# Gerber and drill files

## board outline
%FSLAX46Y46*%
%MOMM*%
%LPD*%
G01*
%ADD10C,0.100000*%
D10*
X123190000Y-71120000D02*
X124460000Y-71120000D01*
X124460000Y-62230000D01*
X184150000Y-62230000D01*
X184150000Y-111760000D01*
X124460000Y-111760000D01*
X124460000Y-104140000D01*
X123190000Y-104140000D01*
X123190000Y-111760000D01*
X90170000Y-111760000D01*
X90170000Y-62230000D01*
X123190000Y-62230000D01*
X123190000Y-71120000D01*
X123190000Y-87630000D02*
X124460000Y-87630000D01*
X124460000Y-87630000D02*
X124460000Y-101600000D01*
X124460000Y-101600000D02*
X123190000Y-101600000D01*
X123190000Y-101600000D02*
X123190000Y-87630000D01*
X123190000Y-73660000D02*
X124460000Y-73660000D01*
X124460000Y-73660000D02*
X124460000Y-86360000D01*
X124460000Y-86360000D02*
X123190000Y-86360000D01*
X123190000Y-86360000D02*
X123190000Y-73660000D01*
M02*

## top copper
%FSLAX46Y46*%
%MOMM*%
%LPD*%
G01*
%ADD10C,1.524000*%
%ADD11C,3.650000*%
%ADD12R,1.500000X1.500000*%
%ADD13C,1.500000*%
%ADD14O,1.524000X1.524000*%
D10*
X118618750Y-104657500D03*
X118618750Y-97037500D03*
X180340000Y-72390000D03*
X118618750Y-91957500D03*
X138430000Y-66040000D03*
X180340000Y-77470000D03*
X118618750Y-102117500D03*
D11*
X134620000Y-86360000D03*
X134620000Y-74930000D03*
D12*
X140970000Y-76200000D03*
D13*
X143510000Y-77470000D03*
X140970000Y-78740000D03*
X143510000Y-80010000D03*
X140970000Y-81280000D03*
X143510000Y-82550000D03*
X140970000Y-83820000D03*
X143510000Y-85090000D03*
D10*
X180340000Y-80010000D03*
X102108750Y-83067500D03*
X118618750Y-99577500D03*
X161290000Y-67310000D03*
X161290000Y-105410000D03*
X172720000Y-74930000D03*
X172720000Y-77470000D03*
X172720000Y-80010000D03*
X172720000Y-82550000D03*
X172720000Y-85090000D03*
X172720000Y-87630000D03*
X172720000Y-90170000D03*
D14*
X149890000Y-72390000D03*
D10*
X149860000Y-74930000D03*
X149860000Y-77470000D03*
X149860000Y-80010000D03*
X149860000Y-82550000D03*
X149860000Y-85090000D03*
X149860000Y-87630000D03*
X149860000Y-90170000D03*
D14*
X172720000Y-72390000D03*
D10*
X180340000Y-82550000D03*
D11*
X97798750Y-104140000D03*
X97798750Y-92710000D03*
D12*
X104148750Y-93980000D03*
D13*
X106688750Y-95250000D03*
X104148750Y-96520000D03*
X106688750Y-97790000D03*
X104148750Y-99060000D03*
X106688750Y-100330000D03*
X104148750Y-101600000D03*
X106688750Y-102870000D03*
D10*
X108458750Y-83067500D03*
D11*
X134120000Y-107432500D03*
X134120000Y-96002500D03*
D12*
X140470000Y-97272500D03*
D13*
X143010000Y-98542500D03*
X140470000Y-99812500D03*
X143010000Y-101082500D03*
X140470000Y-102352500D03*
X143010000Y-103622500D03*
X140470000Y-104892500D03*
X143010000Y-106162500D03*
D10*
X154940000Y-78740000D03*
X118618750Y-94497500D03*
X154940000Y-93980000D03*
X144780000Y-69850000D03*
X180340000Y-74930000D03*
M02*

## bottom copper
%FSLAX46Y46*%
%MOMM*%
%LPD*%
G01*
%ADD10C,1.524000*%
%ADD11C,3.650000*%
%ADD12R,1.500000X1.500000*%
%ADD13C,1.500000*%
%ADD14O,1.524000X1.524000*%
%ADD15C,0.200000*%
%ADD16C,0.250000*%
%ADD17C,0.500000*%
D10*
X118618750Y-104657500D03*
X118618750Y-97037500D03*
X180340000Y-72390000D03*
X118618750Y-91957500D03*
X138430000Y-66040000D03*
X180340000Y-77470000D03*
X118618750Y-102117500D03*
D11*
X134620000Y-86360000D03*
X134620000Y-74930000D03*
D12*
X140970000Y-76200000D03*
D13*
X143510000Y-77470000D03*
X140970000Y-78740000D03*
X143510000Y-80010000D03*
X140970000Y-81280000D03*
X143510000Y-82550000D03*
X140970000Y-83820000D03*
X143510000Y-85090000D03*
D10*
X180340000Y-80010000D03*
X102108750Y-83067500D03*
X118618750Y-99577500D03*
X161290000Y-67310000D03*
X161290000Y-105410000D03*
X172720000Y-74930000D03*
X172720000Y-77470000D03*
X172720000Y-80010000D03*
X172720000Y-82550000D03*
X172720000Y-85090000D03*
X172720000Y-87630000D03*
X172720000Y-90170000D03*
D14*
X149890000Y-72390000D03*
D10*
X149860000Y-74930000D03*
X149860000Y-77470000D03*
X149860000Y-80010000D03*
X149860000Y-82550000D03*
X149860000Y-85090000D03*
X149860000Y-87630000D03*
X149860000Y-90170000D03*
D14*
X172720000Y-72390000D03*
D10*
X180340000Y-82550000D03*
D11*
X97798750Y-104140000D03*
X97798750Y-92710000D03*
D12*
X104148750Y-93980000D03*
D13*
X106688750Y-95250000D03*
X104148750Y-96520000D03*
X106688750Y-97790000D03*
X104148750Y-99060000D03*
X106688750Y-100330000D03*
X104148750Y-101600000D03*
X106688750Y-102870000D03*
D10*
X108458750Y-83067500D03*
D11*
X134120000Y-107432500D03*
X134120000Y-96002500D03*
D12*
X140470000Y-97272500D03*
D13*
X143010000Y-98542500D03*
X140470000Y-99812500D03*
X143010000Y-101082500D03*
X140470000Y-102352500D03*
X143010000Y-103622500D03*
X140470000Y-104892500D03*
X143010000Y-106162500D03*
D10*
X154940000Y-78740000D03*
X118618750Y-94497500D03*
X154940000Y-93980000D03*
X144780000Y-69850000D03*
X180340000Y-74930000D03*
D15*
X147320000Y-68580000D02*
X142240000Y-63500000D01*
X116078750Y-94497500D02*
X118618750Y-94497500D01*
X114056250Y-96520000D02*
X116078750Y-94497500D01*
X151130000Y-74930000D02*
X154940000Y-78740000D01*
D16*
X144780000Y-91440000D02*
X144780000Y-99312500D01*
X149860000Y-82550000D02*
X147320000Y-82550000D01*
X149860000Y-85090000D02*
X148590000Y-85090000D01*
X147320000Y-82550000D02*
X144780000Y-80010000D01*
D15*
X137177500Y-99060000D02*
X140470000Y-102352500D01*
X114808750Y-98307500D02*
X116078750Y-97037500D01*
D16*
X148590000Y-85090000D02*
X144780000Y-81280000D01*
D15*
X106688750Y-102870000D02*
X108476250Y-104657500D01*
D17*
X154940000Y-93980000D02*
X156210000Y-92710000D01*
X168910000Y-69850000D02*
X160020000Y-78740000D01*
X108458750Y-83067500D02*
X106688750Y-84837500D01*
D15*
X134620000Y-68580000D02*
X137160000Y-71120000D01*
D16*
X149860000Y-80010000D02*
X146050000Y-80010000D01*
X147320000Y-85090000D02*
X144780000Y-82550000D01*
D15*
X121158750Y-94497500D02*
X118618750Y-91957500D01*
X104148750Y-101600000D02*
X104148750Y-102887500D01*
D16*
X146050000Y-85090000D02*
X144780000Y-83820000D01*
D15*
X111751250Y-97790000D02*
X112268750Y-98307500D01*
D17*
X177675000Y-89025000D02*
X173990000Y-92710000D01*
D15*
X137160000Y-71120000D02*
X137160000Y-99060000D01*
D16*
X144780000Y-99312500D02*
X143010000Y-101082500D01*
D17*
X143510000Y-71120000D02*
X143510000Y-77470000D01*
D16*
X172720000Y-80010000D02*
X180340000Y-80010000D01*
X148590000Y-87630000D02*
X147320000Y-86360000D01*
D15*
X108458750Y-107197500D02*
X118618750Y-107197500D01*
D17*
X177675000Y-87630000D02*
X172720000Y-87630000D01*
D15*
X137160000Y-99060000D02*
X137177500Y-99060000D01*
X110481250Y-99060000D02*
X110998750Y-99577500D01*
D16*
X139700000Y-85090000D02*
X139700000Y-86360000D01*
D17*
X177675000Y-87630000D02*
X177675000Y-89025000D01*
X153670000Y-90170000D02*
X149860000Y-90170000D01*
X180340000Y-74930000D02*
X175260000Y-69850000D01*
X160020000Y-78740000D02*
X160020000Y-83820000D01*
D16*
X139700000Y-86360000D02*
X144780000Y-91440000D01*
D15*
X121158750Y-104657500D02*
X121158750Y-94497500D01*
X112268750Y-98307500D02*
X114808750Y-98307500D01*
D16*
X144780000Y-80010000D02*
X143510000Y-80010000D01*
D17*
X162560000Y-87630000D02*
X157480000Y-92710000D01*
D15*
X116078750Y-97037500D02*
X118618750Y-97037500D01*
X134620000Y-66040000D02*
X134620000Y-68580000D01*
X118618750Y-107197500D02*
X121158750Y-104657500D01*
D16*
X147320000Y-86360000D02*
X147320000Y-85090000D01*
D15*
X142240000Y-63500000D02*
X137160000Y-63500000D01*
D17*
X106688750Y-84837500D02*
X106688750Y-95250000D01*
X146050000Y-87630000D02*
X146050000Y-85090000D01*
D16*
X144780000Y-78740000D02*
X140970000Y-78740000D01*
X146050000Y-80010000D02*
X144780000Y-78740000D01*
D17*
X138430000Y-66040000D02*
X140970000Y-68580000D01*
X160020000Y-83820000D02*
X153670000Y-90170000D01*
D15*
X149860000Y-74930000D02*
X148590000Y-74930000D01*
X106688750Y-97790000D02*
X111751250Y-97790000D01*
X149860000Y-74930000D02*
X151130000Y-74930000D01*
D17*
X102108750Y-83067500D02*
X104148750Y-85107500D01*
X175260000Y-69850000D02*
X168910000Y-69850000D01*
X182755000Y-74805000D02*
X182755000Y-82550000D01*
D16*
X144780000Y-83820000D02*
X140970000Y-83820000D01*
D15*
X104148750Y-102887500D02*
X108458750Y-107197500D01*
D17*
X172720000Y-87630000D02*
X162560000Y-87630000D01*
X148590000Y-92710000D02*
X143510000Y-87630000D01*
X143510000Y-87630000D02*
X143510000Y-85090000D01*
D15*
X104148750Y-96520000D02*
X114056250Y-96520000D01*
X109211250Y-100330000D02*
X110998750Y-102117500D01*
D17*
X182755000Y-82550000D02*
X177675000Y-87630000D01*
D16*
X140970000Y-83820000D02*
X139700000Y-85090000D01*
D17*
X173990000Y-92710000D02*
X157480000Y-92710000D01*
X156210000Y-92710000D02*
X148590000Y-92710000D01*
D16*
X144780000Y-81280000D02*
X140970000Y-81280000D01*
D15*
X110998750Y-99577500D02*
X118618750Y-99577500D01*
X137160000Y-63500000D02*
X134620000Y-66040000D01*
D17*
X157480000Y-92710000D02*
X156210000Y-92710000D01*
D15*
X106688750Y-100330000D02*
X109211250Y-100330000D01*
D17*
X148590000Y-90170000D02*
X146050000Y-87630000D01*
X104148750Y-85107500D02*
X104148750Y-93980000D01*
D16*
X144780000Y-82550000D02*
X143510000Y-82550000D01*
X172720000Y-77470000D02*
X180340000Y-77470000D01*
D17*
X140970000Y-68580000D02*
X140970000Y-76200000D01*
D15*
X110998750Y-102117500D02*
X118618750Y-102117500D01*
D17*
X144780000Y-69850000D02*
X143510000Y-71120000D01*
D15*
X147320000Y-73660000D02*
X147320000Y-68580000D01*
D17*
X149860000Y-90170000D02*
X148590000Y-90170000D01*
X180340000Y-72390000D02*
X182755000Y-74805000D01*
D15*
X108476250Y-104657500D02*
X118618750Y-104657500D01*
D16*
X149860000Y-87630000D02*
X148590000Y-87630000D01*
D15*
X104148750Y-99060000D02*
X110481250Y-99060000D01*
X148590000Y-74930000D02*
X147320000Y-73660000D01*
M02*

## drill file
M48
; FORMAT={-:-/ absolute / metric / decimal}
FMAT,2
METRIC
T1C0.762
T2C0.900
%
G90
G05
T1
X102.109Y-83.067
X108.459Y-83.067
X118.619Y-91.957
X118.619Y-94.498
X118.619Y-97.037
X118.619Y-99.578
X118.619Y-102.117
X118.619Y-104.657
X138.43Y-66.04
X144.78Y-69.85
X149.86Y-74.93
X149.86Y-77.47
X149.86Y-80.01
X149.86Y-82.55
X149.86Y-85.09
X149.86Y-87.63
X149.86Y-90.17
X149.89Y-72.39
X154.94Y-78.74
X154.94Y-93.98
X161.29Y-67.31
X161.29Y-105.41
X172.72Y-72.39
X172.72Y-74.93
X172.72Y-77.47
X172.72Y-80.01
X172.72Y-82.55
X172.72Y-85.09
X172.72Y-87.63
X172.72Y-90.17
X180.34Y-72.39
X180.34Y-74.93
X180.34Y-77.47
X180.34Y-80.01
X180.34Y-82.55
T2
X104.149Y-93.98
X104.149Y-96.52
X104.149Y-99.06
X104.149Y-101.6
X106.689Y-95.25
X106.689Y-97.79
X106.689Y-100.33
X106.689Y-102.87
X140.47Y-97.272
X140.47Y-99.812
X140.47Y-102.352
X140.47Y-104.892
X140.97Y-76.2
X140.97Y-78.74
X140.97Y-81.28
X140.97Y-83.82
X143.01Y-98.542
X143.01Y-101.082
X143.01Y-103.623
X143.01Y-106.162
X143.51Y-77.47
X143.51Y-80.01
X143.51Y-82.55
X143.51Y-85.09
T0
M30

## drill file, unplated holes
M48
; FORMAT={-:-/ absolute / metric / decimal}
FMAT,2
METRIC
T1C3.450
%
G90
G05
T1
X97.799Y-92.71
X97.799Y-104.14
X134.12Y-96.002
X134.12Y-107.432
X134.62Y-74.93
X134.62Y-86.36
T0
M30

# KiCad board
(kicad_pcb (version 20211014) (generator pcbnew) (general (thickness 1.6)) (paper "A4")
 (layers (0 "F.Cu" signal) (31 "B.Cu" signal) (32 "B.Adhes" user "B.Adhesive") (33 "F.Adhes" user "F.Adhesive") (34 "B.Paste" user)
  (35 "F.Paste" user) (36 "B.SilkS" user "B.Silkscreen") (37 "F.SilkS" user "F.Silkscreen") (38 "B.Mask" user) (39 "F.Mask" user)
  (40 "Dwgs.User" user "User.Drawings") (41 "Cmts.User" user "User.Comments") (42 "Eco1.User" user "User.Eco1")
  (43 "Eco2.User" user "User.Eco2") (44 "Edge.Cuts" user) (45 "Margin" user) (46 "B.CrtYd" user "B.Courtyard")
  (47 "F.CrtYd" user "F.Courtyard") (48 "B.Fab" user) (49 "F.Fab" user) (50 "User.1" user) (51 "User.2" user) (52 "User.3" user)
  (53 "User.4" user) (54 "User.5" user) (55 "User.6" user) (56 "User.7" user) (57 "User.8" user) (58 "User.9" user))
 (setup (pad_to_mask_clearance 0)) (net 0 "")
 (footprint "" (layer "F.Cu") (at 118.61875 104.6575)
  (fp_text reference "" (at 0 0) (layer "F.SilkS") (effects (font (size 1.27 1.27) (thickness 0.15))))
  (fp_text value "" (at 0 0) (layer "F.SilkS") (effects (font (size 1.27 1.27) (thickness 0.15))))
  (pad "1" thru_hole circle (at 0 0) (size 1.524 1.524) (drill 0.762) (layers *.Cu *.Mask)))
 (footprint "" (layer "F.Cu") (at 118.61875 97.0375)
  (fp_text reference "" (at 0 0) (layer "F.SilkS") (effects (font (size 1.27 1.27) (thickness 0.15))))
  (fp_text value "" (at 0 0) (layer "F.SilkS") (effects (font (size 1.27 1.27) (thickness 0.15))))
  (pad "1" thru_hole circle (at 0 0) (size 1.524 1.524) (drill 0.762) (layers *.Cu *.Mask)))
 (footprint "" (layer "F.Cu") (at 180.34 72.39)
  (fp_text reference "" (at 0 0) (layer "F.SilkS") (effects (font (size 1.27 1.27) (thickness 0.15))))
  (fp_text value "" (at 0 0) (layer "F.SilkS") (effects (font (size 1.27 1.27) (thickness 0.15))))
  (pad "1" thru_hole circle (at 0 0) (size 1.524 1.524) (drill 0.762) (layers *.Cu *.Mask)))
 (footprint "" (layer "F.Cu") (at 118.61875 91.9575)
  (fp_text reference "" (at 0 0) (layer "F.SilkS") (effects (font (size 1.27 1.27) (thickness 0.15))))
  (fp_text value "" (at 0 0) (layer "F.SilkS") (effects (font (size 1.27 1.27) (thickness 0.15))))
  (pad "1" thru_hole circle (at 0 0) (size 1.524 1.524) (drill 0.762) (layers *.Cu *.Mask)))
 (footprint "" (layer "F.Cu") (at 138.43 66.04)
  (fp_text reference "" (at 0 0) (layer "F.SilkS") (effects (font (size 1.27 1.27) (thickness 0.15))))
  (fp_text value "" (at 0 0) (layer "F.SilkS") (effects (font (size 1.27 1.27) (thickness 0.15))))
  (pad "1" thru_hole circle (at 0 0) (size 1.524 1.524) (drill 0.762) (layers *.Cu *.Mask)))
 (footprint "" (layer "F.Cu") (at 180.34 77.47)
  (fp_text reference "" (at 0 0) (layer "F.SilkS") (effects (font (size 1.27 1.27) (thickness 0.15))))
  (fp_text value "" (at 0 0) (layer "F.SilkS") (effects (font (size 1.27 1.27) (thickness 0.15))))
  (pad "1" thru_hole circle (at 0 0) (size 1.524 1.524) (drill 0.762) (layers *.Cu *.Mask)))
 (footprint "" (layer "F.Cu") (at 118.61875 102.1175)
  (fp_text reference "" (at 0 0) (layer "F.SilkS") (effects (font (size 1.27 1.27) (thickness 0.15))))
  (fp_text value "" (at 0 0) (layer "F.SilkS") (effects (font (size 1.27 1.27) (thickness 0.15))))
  (pad "1" thru_hole circle (at 0 0) (size 1.524 1.524) (drill 0.762) (layers *.Cu *.Mask)))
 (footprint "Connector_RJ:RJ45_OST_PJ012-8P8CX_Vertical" (layer "F.Cu") (at 140.97 76.2 -90)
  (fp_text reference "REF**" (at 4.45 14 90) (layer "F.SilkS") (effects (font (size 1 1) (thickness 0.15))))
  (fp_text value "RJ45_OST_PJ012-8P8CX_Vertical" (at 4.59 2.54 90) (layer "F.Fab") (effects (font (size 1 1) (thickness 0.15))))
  (pad "" np_thru_hole circle (at 10.16 6.35 270) (size 3.65 3.65) (drill 3.45) (layers *.Cu *.SilkS *.Mask))
  (pad "" np_thru_hole circle (at -1.27 6.35 270) (size 3.65 3.65) (drill 3.45) (layers F&B.Cu *.SilkS *.Mask))
  (pad "1" thru_hole rect (at 0 0 270) (size 1.5 1.5) (drill 0.9) (layers *.Cu *.Mask))
  (pad "2" thru_hole circle (at 1.27 -2.54 270) (size 1.5 1.5) (drill 0.9) (layers *.Cu *.Mask))
  (pad "3" thru_hole circle (at 2.54 0 270) (size 1.5 1.5) (drill 0.9) (layers *.Cu *.Mask))
  (pad "4" thru_hole circle (at 3.81 -2.54 270) (size 1.5 1.5) (drill 0.9) (layers *.Cu *.Mask))
  (pad "5" thru_hole circle (at 5.08 0 270) (size 1.5 1.5) (drill 0.9) (layers *.Cu *.Mask))
  (pad "6" thru_hole circle (at 6.35 -2.54 270) (size 1.5 1.5) (drill 0.9) (layers *.Cu *.Mask))
  (pad "7" thru_hole circle (at 7.62 0 270) (size 1.5 1.5) (drill 0.9) (layers *.Cu *.Mask))
  (pad "8" thru_hole circle (at 8.89 -2.54 270) (size 1.5 1.5) (drill 0.9) (layers *.Cu *.Mask)))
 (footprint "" (layer "F.Cu") (at 180.34 80.01)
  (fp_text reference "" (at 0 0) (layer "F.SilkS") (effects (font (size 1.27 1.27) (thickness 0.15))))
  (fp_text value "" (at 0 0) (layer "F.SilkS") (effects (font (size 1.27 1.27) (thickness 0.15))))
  (pad "1" thru_hole circle (at 0 0) (size 1.524 1.524) (drill 0.762) (layers *.Cu *.Mask)))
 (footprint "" (layer "F.Cu") (at 102.10875 83.0675)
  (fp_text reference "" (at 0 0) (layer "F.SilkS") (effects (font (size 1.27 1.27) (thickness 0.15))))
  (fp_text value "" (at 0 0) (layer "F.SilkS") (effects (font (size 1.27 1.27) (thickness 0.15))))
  (pad "1" thru_hole circle (at 0 0) (size 1.524 1.524) (drill 0.762) (layers *.Cu *.Mask)))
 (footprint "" (layer "F.Cu") (at 118.61875 99.5775)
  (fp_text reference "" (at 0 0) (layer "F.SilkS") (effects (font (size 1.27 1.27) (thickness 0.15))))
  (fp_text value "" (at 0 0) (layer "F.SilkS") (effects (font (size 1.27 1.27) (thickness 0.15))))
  (pad "1" thru_hole circle (at 0 0) (size 1.524 1.524) (drill 0.762) (layers *.Cu *.Mask)))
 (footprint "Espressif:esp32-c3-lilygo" (layer "F.Cu") (at 148.59 64.77)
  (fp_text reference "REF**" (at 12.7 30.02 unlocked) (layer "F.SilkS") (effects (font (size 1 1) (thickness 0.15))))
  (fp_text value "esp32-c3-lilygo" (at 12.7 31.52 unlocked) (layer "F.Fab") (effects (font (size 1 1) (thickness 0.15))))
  (pad "1" thru_hole circle (at 12.7 2.54) (size 1.524 1.524) (drill 0.762) (layers *.Cu *.Mask))
  (pad "2" thru_hole circle (at 12.7 40.64) (size 1.524 1.524) (drill 0.762) (layers *.Cu *.Mask))
  (pad "5" thru_hole circle (at 24.13 10.16) (size 1.524 1.524) (drill 0.762) (layers *.Cu *.Mask))
  (pad "6" thru_hole circle (at 24.13 12.7) (size 1.524 1.524) (drill 0.762) (layers *.Cu *.Mask))
  (pad "7" thru_hole circle (at 24.13 15.24) (size 1.524 1.524) (drill 0.762) (layers *.Cu *.Mask))
  (pad "8" thru_hole circle (at 24.13 17.78) (size 1.524 1.524) (drill 0.762) (layers *.Cu *.Mask))
  (pad "9" thru_hole circle (at 24.13 20.32) (size 1.524 1.524) (drill 0.762) (layers *.Cu *.Mask))
  (pad "10" thru_hole circle (at 24.13 22.86) (size 1.524 1.524) (drill 0.762) (layers *.Cu *.Mask))
  (pad "11" thru_hole circle (at 24.13 25.4) (size 1.524 1.524) (drill 0.762) (layers *.Cu *.Mask))
  (pad "12" thru_hole oval (at 1.3 7.62) (size 1.524 1.524) (drill 0.762) (layers *.Cu *.Mask))
  (pad "13" thru_hole circle (at 1.27 10.16) (size 1.524 1.524) (drill 0.762) (layers *.Cu *.Mask))
  (pad "14" thru_hole circle (at 1.27 12.7) (size 1.524 1.524) (drill 0.762) (layers *.Cu *.Mask))
  (pad "15" thru_hole circle (at 1.27 15.24) (size 1.524 1.524) (drill 0.762) (layers *.Cu *.Mask))
  (pad "16" thru_hole circle (at 1.27 17.78) (size 1.524 1.524) (drill 0.762) (layers *.Cu *.Mask))
  (pad "17" thru_hole circle (at 1.27 20.32) (size 1.524 1.524) (drill 0.762) (layers *.Cu *.Mask))
  (pad "18" thru_hole circle (at 1.27 22.86) (size 1.524 1.524) (drill 0.762) (layers *.Cu *.Mask))
  (pad "19" thru_hole circle (at 1.27 25.4) (size 1.524 1.524) (drill 0.762) (layers *.Cu *.Mask))
  (pad "20" thru_hole oval (at 24.13 7.62) (size 1.524 1.524) (drill 0.762) (layers *.Cu *.Mask)))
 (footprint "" (layer "F.Cu") (at 180.34 82.55)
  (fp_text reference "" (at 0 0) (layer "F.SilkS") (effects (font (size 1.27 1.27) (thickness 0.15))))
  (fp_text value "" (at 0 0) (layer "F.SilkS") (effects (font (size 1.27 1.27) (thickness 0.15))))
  (pad "1" thru_hole circle (at 0 0) (size 1.524 1.524) (drill 0.762) (layers *.Cu *.Mask)))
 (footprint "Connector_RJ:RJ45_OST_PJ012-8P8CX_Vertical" (layer "F.Cu") (at 104.14875 93.98 -90)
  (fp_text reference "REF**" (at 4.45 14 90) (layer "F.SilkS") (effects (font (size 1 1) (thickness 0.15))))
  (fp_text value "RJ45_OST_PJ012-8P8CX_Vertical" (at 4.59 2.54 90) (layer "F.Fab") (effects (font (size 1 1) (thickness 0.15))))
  (pad "" np_thru_hole circle (at 10.16 6.35 270) (size 3.65 3.65) (drill 3.45) (layers *.Cu *.SilkS *.Mask))
  (pad "" np_thru_hole circle (at -1.27 6.35 270) (size 3.65 3.65) (drill 3.45) (layers *.Cu *.SilkS *.Mask))
  (pad "1" thru_hole rect (at 0 0 270) (size 1.5 1.5) (drill 0.9) (layers *.Cu *.Mask))
  (pad "2" thru_hole circle (at 1.27 -2.54 270) (size 1.5 1.5) (drill 0.9) (layers *.Cu *.Mask))
  (pad "3" thru_hole circle (at 2.54 0 270) (size 1.5 1.5) (drill 0.9) (layers *.Cu *.Mask))
  (pad "4" thru_hole circle (at 3.81 -2.54 270) (size 1.5 1.5) (drill 0.9) (layers *.Cu *.Mask))
  (pad "5" thru_hole circle (at 5.08 0 270) (size 1.5 1.5) (drill 0.9) (layers *.Cu *.Mask))
  (pad "6" thru_hole circle (at 6.35 -2.54 270) (size 1.5 1.5) (drill 0.9) (layers *.Cu *.Mask))
  (pad "7" thru_hole circle (at 7.62 0 270) (size 1.5 1.5) (drill 0.9) (layers *.Cu *.Mask))
  (pad "8" thru_hole circle (at 8.89 -2.54 270) (size 1.5 1.5) (drill 0.9) (layers *.Cu *.Mask)))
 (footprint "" (layer "F.Cu") (at 108.45875 83.0675)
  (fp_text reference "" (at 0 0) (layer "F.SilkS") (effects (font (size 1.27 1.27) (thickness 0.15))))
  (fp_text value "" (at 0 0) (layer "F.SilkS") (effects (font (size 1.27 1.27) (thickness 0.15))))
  (pad "1" thru_hole circle (at 0 0) (size 1.524 1.524) (drill 0.762) (layers *.Cu *.Mask)))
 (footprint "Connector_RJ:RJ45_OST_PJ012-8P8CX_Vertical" (layer "F.Cu") (at 140.47 97.2725 -90)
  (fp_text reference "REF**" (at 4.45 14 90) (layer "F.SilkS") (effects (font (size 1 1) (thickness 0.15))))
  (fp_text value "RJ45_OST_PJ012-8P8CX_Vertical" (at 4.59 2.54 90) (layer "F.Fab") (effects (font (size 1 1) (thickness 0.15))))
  (pad "" np_thru_hole circle (at 10.16 6.35 270) (size 3.65 3.65) (drill 3.45) (layers *.Cu *.SilkS *.Mask))
  (pad "" np_thru_hole circle (at -1.27 6.35 270) (size 3.65 3.65) (drill 3.45) (layers *.Cu *.SilkS *.Mask))
  (pad "1" thru_hole rect (at 0 0 270) (size 1.5 1.5) (drill 0.9) (layers *.Cu *.Mask))
  (pad "2" thru_hole circle (at 1.27 -2.54 270) (size 1.5 1.5) (drill 0.9) (layers *.Cu *.Mask))
  (pad "3" thru_hole circle (at 2.54 0 270) (size 1.5 1.5) (drill 0.9) (layers *.Cu *.Mask))
  (pad "4" thru_hole circle (at 3.81 -2.54 270) (size 1.5 1.5) (drill 0.9) (layers *.Cu *.Mask))
  (pad "5" thru_hole circle (at 5.08 0 270) (size 1.5 1.5) (drill 0.9) (layers *.Cu *.Mask))
  (pad "6" thru_hole circle (at 6.35 -2.54 270) (size 1.5 1.5) (drill 0.9) (layers *.Cu *.Mask))
  (pad "7" thru_hole circle (at 7.62 0 270) (size 1.5 1.5) (drill 0.9) (layers *.Cu *.Mask))
  (pad "8" thru_hole circle (at 8.89 -2.54 270) (size 1.5 1.5) (drill 0.9) (layers *.Cu *.Mask)))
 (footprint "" (layer "F.Cu") (at 154.94 78.74)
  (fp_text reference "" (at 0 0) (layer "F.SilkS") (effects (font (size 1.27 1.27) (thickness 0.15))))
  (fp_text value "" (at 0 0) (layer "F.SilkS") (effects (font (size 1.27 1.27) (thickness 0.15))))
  (pad "1" thru_hole circle (at 0 0) (size 1.524 1.524) (drill 0.762) (layers *.Cu *.Mask)))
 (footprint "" (layer "F.Cu") (at 118.61875 94.4975)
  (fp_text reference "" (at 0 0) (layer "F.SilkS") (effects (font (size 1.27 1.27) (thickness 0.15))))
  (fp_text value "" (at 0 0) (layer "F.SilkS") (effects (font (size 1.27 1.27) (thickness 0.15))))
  (pad "1" thru_hole circle (at 0 0) (size 1.524 1.524) (drill 0.762) (layers *.Cu *.Mask)))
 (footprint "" (layer "F.Cu") (at 154.94 93.98)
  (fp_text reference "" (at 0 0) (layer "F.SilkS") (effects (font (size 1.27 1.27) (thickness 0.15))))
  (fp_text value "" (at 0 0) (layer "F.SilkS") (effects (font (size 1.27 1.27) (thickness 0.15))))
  (pad "1" thru_hole circle (at 0 0) (size 1.524 1.524) (drill 0.762) (layers *.Cu *.Mask)))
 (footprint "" (layer "F.Cu") (at 144.78 69.85)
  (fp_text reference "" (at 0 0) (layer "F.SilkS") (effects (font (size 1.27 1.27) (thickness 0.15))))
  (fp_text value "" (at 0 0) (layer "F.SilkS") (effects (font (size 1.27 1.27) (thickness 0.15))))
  (pad "1" thru_hole circle (at 0 0) (size 1.524 1.524) (drill 0.762) (layers *.Cu *.Mask)))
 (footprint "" (layer "F.Cu") (at 180.34 74.93)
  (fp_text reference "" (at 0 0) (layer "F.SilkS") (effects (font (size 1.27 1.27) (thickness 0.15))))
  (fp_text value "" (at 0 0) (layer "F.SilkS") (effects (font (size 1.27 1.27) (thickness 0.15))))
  (pad "1" thru_hole circle (at 0 0) (size 1.524 1.524) (drill 0.762) (layers *.Cu *.Mask)))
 (gr_poly
  (pts (xy 123.19 71.12) (xy 124.46 71.12) (xy 124.46 62.23) (xy 184.15 62.23) (xy 184.15 111.76) (xy 124.46 111.76) (xy 124.46 104.14)
   (xy 123.19 104.14) (xy 123.19 111.76) (xy 90.17 111.76) (xy 90.17 62.23) (xy 123.19 62.23))
  (layer "Edge.Cuts") (width 0.1) (fill none))
 (gr_rect (start 123.19 87.63) (end 124.46 101.6) (layer "Edge.Cuts") (width 0.1) (fill none))
 (gr_rect (start 123.19 73.66) (end 124.46 86.36) (layer "Edge.Cuts") (width 0.1) (fill none))
 (segment (start 147.32 68.58) (end 142.24 63.5) (width 0.2) (layer "B.Cu") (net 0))
 (segment (start 116.07875 94.4975) (end 118.61875 94.4975) (width 0.2) (layer "B.Cu") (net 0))
 (segment (start 114.05625 96.52) (end 116.07875 94.4975) (width 0.2) (layer "B.Cu") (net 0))
 (segment (start 151.13 74.93) (end 154.94 78.74) (width 0.2) (layer "B.Cu") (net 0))
 (segment (start 144.78 91.44) (end 144.78 99.3125) (width 0.25) (layer "B.Cu") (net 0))
 (segment (start 149.86 82.55) (end 147.32 82.55) (width 0.25) (layer "B.Cu") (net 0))
 (segment (start 149.86 85.09) (end 148.59 85.09) (width 0.25) (layer "B.Cu") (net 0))
 (segment (start 147.32 82.55) (end 144.78 80.01) (width 0.25) (layer "B.Cu") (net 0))
 (segment (start 137.1775 99.06) (end 140.47 102.3525) (width 0.2) (layer "B.Cu") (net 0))
 (segment (start 114.80875 98.3075) (end 116.07875 97.0375) (width 0.2) (layer "B.Cu") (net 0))
 (segment (start 148.59 85.09) (end 144.78 81.28) (width 0.25) (layer "B.Cu") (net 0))
 (segment (start 106.68875 102.87) (end 108.47625 104.6575) (width 0.2) (layer "B.Cu") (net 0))
 (segment (start 154.94 93.98) (end 156.21 92.71) (width 0.5) (layer "B.Cu") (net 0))
 (segment (start 168.91 69.85) (end 160.02 78.74) (width 0.5) (layer "B.Cu") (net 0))
 (segment (start 108.45875 83.0675) (end 106.68875 84.8375) (width 0.5) (layer "B.Cu") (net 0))
 (segment (start 134.62 68.58) (end 137.16 71.12) (width 0.2) (layer "B.Cu") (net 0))
 (segment (start 149.86 80.01) (end 146.05 80.01) (width 0.25) (layer "B.Cu") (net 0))
 (segment (start 147.32 85.09) (end 144.78 82.55) (width 0.25) (layer "B.Cu") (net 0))
 (segment (start 121.15875 94.4975) (end 118.61875 91.9575) (width 0.2) (layer "B.Cu") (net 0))
 (segment (start 104.14875 101.6) (end 104.14875 102.8875) (width 0.2) (layer "B.Cu") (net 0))
 (segment (start 146.05 85.09) (end 144.78 83.82) (width 0.25) (layer "B.Cu") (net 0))
 (segment (start 111.75125 97.79) (end 112.26875 98.3075) (width 0.2) (layer "B.Cu") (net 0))
 (segment (start 177.675 89.025) (end 173.99 92.71) (width 0.5) (layer "B.Cu") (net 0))
 (segment (start 137.16 71.12) (end 137.16 99.06) (width 0.2) (layer "B.Cu") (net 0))
 (segment (start 144.78 99.3125) (end 143.01 101.0825) (width 0.25) (layer "B.Cu") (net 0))
 (segment (start 143.51 71.12) (end 143.51 77.47) (width 0.5) (layer "B.Cu") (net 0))
 (segment (start 172.72 80.01) (end 180.34 80.01) (width 0.25) (layer "B.Cu") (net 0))
 (segment (start 148.59 87.63) (end 147.32 86.36) (width 0.25) (layer "B.Cu") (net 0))
 (segment (start 108.45875 107.1975) (end 118.61875 107.1975) (width 0.2) (layer "B.Cu") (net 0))
 (segment (start 177.675 87.63) (end 172.72 87.63) (width 0.5) (layer "B.Cu") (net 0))
 (segment (start 137.16 99.06) (end 137.1775 99.06) (width 0.2) (layer "B.Cu") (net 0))
 (segment (start 110.48125 99.06) (end 110.99875 99.5775) (width 0.2) (layer "B.Cu") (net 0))
 (segment (start 139.7 85.09) (end 139.7 86.36) (width 0.25) (layer "B.Cu") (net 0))
 (segment (start 177.675 87.63) (end 177.675 89.025) (width 0.5) (layer "B.Cu") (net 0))
 (segment (start 153.67 90.17) (end 149.86 90.17) (width 0.5) (layer "B.Cu") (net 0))
 (segment (start 180.34 74.93) (end 175.26 69.85) (width 0.5) (layer "B.Cu") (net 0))
 (segment (start 160.02 78.74) (end 160.02 83.82) (width 0.5) (layer "B.Cu") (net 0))
 (segment (start 139.7 86.36) (end 144.78 91.44) (width 0.25) (layer "B.Cu") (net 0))
 (segment (start 121.15875 104.6575) (end 121.15875 94.4975) (width 0.2) (layer "B.Cu") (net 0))
 (segment (start 112.26875 98.3075) (end 114.80875 98.3075) (width 0.2) (layer "B.Cu") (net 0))
 (segment (start 144.78 80.01) (end 143.51 80.01) (width 0.25) (layer "B.Cu") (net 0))
 (segment (start 162.56 87.63) (end 157.48 92.71) (width 0.5) (layer "B.Cu") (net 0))
 (segment (start 116.07875 97.0375) (end 118.61875 97.0375) (width 0.2) (layer "B.Cu") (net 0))
 (segment (start 134.62 66.04) (end 134.62 68.58) (width 0.2) (layer "B.Cu") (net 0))
 (segment (start 118.61875 107.1975) (end 121.15875 104.6575) (width 0.2) (layer "B.Cu") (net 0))
 (segment (start 147.32 86.36) (end 147.32 85.09) (width 0.25) (layer "B.Cu") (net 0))
 (segment (start 142.24 63.5) (end 137.16 63.5) (width 0.2) (layer "B.Cu") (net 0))
 (segment (start 106.68875 84.8375) (end 106.68875 95.25) (width 0.5) (layer "B.Cu") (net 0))
 (segment (start 146.05 87.63) (end 146.05 85.09) (width 0.5) (layer "B.Cu") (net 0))
 (segment (start 144.78 78.74) (end 140.97 78.74) (width 0.25) (layer "B.Cu") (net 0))
 (segment (start 146.05 80.01) (end 144.78 78.74) (width 0.25) (layer "B.Cu") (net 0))
 (segment (start 138.43 66.04) (end 140.97 68.58) (width 0.5) (layer "B.Cu") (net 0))
 (segment (start 160.02 83.82) (end 153.67 90.17) (width 0.5) (layer "B.Cu") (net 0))
 (segment (start 149.86 74.93) (end 148.59 74.93) (width 0.2) (layer "B.Cu") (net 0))
 (segment (start 106.68875 97.79) (end 111.75125 97.79) (width 0.2) (layer "B.Cu") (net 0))
 (segment (start 149.86 74.93) (end 151.13 74.93) (width 0.2) (layer "B.Cu") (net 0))
 (segment (start 102.10875 83.0675) (end 104.14875 85.1075) (width 0.5) (layer "B.Cu") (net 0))
 (segment (start 175.26 69.85) (end 168.91 69.85) (width 0.5) (layer "B.Cu") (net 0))
 (segment (start 182.755 74.805) (end 182.755 82.55) (width 0.5) (layer "B.Cu") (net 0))
 (segment (start 144.78 83.82) (end 140.97 83.82) (width 0.25) (layer "B.Cu") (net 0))
 (segment (start 104.14875 102.8875) (end 108.45875 107.1975) (width 0.2) (layer "B.Cu") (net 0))
 (segment (start 172.72 87.63) (end 162.56 87.63) (width 0.5) (layer "B.Cu") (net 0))
 (segment (start 148.59 92.71) (end 143.51 87.63) (width 0.5) (layer "B.Cu") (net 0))
 (segment (start 143.51 87.63) (end 143.51 85.09) (width 0.5) (layer "B.Cu") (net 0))
 (segment (start 104.14875 96.52) (end 114.05625 96.52) (width 0.2) (layer "B.Cu") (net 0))
 (segment (start 109.21125 100.33) (end 110.99875 102.1175) (width 0.2) (layer "B.Cu") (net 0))
 (segment (start 182.755 82.55) (end 177.675 87.63) (width 0.5) (layer "B.Cu") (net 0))
 (segment (start 140.97 83.82) (end 139.7 85.09) (width 0.25) (layer "B.Cu") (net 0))
 (segment (start 173.99 92.71) (end 157.48 92.71) (width 0.5) (layer "B.Cu") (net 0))
 (segment (start 156.21 92.71) (end 148.59 92.71) (width 0.5) (layer "B.Cu") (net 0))
 (segment (start 144.78 81.28) (end 140.97 81.28) (width 0.25) (layer "B.Cu") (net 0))
 (segment (start 110.99875 99.5775) (end 118.61875 99.5775) (width 0.2) (layer "B.Cu") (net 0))
 (segment (start 137.16 63.5) (end 134.62 66.04) (width 0.2) (layer "B.Cu") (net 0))
 (segment (start 157.48 92.71) (end 156.21 92.71) (width 0.5) (layer "B.Cu") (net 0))
 (segment (start 106.68875 100.33) (end 109.21125 100.33) (width 0.2) (layer "B.Cu") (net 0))
 (segment (start 148.59 90.17) (end 146.05 87.63) (width 0.5) (layer "B.Cu") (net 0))
 (segment (start 104.14875 85.1075) (end 104.14875 93.98) (width 0.5) (layer "B.Cu") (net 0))
 (segment (start 144.78 82.55) (end 143.51 82.55) (width 0.25) (layer "B.Cu") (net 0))
 (segment (start 172.72 77.47) (end 180.34 77.47) (width 0.25) (layer "B.Cu") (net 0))
 (segment (start 140.97 68.58) (end 140.97 76.2) (width 0.5) (layer "B.Cu") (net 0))
 (segment (start 110.99875 102.1175) (end 118.61875 102.1175) (width 0.2) (layer "B.Cu") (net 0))
 (segment (start 144.78 69.85) (end 143.51 71.12) (width 0.5) (layer "B.Cu") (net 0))
 (segment (start 147.32 73.66) (end 147.32 68.58) (width 0.2) (layer "B.Cu") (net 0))
 (segment (start 149.86 90.17) (end 148.59 90.17) (width 0.5) (layer "B.Cu") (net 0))
 (segment (start 180.34 72.39) (end 182.755 74.805) (width 0.5) (layer "B.Cu") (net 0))
 (segment (start 108.47625 104.6575) (end 118.61875 104.6575) (width 0.2) (layer "B.Cu") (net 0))
 (segment (start 149.86 87.63) (end 148.59 87.63) (width 0.25) (layer "B.Cu") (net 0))
 (segment (start 104.14875 99.06) (end 110.48125 99.06) (width 0.2) (layer "B.Cu") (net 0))
 (segment (start 148.59 74.93) (end 147.32 73.66) (width 0.2) (layer "B.Cu") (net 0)))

